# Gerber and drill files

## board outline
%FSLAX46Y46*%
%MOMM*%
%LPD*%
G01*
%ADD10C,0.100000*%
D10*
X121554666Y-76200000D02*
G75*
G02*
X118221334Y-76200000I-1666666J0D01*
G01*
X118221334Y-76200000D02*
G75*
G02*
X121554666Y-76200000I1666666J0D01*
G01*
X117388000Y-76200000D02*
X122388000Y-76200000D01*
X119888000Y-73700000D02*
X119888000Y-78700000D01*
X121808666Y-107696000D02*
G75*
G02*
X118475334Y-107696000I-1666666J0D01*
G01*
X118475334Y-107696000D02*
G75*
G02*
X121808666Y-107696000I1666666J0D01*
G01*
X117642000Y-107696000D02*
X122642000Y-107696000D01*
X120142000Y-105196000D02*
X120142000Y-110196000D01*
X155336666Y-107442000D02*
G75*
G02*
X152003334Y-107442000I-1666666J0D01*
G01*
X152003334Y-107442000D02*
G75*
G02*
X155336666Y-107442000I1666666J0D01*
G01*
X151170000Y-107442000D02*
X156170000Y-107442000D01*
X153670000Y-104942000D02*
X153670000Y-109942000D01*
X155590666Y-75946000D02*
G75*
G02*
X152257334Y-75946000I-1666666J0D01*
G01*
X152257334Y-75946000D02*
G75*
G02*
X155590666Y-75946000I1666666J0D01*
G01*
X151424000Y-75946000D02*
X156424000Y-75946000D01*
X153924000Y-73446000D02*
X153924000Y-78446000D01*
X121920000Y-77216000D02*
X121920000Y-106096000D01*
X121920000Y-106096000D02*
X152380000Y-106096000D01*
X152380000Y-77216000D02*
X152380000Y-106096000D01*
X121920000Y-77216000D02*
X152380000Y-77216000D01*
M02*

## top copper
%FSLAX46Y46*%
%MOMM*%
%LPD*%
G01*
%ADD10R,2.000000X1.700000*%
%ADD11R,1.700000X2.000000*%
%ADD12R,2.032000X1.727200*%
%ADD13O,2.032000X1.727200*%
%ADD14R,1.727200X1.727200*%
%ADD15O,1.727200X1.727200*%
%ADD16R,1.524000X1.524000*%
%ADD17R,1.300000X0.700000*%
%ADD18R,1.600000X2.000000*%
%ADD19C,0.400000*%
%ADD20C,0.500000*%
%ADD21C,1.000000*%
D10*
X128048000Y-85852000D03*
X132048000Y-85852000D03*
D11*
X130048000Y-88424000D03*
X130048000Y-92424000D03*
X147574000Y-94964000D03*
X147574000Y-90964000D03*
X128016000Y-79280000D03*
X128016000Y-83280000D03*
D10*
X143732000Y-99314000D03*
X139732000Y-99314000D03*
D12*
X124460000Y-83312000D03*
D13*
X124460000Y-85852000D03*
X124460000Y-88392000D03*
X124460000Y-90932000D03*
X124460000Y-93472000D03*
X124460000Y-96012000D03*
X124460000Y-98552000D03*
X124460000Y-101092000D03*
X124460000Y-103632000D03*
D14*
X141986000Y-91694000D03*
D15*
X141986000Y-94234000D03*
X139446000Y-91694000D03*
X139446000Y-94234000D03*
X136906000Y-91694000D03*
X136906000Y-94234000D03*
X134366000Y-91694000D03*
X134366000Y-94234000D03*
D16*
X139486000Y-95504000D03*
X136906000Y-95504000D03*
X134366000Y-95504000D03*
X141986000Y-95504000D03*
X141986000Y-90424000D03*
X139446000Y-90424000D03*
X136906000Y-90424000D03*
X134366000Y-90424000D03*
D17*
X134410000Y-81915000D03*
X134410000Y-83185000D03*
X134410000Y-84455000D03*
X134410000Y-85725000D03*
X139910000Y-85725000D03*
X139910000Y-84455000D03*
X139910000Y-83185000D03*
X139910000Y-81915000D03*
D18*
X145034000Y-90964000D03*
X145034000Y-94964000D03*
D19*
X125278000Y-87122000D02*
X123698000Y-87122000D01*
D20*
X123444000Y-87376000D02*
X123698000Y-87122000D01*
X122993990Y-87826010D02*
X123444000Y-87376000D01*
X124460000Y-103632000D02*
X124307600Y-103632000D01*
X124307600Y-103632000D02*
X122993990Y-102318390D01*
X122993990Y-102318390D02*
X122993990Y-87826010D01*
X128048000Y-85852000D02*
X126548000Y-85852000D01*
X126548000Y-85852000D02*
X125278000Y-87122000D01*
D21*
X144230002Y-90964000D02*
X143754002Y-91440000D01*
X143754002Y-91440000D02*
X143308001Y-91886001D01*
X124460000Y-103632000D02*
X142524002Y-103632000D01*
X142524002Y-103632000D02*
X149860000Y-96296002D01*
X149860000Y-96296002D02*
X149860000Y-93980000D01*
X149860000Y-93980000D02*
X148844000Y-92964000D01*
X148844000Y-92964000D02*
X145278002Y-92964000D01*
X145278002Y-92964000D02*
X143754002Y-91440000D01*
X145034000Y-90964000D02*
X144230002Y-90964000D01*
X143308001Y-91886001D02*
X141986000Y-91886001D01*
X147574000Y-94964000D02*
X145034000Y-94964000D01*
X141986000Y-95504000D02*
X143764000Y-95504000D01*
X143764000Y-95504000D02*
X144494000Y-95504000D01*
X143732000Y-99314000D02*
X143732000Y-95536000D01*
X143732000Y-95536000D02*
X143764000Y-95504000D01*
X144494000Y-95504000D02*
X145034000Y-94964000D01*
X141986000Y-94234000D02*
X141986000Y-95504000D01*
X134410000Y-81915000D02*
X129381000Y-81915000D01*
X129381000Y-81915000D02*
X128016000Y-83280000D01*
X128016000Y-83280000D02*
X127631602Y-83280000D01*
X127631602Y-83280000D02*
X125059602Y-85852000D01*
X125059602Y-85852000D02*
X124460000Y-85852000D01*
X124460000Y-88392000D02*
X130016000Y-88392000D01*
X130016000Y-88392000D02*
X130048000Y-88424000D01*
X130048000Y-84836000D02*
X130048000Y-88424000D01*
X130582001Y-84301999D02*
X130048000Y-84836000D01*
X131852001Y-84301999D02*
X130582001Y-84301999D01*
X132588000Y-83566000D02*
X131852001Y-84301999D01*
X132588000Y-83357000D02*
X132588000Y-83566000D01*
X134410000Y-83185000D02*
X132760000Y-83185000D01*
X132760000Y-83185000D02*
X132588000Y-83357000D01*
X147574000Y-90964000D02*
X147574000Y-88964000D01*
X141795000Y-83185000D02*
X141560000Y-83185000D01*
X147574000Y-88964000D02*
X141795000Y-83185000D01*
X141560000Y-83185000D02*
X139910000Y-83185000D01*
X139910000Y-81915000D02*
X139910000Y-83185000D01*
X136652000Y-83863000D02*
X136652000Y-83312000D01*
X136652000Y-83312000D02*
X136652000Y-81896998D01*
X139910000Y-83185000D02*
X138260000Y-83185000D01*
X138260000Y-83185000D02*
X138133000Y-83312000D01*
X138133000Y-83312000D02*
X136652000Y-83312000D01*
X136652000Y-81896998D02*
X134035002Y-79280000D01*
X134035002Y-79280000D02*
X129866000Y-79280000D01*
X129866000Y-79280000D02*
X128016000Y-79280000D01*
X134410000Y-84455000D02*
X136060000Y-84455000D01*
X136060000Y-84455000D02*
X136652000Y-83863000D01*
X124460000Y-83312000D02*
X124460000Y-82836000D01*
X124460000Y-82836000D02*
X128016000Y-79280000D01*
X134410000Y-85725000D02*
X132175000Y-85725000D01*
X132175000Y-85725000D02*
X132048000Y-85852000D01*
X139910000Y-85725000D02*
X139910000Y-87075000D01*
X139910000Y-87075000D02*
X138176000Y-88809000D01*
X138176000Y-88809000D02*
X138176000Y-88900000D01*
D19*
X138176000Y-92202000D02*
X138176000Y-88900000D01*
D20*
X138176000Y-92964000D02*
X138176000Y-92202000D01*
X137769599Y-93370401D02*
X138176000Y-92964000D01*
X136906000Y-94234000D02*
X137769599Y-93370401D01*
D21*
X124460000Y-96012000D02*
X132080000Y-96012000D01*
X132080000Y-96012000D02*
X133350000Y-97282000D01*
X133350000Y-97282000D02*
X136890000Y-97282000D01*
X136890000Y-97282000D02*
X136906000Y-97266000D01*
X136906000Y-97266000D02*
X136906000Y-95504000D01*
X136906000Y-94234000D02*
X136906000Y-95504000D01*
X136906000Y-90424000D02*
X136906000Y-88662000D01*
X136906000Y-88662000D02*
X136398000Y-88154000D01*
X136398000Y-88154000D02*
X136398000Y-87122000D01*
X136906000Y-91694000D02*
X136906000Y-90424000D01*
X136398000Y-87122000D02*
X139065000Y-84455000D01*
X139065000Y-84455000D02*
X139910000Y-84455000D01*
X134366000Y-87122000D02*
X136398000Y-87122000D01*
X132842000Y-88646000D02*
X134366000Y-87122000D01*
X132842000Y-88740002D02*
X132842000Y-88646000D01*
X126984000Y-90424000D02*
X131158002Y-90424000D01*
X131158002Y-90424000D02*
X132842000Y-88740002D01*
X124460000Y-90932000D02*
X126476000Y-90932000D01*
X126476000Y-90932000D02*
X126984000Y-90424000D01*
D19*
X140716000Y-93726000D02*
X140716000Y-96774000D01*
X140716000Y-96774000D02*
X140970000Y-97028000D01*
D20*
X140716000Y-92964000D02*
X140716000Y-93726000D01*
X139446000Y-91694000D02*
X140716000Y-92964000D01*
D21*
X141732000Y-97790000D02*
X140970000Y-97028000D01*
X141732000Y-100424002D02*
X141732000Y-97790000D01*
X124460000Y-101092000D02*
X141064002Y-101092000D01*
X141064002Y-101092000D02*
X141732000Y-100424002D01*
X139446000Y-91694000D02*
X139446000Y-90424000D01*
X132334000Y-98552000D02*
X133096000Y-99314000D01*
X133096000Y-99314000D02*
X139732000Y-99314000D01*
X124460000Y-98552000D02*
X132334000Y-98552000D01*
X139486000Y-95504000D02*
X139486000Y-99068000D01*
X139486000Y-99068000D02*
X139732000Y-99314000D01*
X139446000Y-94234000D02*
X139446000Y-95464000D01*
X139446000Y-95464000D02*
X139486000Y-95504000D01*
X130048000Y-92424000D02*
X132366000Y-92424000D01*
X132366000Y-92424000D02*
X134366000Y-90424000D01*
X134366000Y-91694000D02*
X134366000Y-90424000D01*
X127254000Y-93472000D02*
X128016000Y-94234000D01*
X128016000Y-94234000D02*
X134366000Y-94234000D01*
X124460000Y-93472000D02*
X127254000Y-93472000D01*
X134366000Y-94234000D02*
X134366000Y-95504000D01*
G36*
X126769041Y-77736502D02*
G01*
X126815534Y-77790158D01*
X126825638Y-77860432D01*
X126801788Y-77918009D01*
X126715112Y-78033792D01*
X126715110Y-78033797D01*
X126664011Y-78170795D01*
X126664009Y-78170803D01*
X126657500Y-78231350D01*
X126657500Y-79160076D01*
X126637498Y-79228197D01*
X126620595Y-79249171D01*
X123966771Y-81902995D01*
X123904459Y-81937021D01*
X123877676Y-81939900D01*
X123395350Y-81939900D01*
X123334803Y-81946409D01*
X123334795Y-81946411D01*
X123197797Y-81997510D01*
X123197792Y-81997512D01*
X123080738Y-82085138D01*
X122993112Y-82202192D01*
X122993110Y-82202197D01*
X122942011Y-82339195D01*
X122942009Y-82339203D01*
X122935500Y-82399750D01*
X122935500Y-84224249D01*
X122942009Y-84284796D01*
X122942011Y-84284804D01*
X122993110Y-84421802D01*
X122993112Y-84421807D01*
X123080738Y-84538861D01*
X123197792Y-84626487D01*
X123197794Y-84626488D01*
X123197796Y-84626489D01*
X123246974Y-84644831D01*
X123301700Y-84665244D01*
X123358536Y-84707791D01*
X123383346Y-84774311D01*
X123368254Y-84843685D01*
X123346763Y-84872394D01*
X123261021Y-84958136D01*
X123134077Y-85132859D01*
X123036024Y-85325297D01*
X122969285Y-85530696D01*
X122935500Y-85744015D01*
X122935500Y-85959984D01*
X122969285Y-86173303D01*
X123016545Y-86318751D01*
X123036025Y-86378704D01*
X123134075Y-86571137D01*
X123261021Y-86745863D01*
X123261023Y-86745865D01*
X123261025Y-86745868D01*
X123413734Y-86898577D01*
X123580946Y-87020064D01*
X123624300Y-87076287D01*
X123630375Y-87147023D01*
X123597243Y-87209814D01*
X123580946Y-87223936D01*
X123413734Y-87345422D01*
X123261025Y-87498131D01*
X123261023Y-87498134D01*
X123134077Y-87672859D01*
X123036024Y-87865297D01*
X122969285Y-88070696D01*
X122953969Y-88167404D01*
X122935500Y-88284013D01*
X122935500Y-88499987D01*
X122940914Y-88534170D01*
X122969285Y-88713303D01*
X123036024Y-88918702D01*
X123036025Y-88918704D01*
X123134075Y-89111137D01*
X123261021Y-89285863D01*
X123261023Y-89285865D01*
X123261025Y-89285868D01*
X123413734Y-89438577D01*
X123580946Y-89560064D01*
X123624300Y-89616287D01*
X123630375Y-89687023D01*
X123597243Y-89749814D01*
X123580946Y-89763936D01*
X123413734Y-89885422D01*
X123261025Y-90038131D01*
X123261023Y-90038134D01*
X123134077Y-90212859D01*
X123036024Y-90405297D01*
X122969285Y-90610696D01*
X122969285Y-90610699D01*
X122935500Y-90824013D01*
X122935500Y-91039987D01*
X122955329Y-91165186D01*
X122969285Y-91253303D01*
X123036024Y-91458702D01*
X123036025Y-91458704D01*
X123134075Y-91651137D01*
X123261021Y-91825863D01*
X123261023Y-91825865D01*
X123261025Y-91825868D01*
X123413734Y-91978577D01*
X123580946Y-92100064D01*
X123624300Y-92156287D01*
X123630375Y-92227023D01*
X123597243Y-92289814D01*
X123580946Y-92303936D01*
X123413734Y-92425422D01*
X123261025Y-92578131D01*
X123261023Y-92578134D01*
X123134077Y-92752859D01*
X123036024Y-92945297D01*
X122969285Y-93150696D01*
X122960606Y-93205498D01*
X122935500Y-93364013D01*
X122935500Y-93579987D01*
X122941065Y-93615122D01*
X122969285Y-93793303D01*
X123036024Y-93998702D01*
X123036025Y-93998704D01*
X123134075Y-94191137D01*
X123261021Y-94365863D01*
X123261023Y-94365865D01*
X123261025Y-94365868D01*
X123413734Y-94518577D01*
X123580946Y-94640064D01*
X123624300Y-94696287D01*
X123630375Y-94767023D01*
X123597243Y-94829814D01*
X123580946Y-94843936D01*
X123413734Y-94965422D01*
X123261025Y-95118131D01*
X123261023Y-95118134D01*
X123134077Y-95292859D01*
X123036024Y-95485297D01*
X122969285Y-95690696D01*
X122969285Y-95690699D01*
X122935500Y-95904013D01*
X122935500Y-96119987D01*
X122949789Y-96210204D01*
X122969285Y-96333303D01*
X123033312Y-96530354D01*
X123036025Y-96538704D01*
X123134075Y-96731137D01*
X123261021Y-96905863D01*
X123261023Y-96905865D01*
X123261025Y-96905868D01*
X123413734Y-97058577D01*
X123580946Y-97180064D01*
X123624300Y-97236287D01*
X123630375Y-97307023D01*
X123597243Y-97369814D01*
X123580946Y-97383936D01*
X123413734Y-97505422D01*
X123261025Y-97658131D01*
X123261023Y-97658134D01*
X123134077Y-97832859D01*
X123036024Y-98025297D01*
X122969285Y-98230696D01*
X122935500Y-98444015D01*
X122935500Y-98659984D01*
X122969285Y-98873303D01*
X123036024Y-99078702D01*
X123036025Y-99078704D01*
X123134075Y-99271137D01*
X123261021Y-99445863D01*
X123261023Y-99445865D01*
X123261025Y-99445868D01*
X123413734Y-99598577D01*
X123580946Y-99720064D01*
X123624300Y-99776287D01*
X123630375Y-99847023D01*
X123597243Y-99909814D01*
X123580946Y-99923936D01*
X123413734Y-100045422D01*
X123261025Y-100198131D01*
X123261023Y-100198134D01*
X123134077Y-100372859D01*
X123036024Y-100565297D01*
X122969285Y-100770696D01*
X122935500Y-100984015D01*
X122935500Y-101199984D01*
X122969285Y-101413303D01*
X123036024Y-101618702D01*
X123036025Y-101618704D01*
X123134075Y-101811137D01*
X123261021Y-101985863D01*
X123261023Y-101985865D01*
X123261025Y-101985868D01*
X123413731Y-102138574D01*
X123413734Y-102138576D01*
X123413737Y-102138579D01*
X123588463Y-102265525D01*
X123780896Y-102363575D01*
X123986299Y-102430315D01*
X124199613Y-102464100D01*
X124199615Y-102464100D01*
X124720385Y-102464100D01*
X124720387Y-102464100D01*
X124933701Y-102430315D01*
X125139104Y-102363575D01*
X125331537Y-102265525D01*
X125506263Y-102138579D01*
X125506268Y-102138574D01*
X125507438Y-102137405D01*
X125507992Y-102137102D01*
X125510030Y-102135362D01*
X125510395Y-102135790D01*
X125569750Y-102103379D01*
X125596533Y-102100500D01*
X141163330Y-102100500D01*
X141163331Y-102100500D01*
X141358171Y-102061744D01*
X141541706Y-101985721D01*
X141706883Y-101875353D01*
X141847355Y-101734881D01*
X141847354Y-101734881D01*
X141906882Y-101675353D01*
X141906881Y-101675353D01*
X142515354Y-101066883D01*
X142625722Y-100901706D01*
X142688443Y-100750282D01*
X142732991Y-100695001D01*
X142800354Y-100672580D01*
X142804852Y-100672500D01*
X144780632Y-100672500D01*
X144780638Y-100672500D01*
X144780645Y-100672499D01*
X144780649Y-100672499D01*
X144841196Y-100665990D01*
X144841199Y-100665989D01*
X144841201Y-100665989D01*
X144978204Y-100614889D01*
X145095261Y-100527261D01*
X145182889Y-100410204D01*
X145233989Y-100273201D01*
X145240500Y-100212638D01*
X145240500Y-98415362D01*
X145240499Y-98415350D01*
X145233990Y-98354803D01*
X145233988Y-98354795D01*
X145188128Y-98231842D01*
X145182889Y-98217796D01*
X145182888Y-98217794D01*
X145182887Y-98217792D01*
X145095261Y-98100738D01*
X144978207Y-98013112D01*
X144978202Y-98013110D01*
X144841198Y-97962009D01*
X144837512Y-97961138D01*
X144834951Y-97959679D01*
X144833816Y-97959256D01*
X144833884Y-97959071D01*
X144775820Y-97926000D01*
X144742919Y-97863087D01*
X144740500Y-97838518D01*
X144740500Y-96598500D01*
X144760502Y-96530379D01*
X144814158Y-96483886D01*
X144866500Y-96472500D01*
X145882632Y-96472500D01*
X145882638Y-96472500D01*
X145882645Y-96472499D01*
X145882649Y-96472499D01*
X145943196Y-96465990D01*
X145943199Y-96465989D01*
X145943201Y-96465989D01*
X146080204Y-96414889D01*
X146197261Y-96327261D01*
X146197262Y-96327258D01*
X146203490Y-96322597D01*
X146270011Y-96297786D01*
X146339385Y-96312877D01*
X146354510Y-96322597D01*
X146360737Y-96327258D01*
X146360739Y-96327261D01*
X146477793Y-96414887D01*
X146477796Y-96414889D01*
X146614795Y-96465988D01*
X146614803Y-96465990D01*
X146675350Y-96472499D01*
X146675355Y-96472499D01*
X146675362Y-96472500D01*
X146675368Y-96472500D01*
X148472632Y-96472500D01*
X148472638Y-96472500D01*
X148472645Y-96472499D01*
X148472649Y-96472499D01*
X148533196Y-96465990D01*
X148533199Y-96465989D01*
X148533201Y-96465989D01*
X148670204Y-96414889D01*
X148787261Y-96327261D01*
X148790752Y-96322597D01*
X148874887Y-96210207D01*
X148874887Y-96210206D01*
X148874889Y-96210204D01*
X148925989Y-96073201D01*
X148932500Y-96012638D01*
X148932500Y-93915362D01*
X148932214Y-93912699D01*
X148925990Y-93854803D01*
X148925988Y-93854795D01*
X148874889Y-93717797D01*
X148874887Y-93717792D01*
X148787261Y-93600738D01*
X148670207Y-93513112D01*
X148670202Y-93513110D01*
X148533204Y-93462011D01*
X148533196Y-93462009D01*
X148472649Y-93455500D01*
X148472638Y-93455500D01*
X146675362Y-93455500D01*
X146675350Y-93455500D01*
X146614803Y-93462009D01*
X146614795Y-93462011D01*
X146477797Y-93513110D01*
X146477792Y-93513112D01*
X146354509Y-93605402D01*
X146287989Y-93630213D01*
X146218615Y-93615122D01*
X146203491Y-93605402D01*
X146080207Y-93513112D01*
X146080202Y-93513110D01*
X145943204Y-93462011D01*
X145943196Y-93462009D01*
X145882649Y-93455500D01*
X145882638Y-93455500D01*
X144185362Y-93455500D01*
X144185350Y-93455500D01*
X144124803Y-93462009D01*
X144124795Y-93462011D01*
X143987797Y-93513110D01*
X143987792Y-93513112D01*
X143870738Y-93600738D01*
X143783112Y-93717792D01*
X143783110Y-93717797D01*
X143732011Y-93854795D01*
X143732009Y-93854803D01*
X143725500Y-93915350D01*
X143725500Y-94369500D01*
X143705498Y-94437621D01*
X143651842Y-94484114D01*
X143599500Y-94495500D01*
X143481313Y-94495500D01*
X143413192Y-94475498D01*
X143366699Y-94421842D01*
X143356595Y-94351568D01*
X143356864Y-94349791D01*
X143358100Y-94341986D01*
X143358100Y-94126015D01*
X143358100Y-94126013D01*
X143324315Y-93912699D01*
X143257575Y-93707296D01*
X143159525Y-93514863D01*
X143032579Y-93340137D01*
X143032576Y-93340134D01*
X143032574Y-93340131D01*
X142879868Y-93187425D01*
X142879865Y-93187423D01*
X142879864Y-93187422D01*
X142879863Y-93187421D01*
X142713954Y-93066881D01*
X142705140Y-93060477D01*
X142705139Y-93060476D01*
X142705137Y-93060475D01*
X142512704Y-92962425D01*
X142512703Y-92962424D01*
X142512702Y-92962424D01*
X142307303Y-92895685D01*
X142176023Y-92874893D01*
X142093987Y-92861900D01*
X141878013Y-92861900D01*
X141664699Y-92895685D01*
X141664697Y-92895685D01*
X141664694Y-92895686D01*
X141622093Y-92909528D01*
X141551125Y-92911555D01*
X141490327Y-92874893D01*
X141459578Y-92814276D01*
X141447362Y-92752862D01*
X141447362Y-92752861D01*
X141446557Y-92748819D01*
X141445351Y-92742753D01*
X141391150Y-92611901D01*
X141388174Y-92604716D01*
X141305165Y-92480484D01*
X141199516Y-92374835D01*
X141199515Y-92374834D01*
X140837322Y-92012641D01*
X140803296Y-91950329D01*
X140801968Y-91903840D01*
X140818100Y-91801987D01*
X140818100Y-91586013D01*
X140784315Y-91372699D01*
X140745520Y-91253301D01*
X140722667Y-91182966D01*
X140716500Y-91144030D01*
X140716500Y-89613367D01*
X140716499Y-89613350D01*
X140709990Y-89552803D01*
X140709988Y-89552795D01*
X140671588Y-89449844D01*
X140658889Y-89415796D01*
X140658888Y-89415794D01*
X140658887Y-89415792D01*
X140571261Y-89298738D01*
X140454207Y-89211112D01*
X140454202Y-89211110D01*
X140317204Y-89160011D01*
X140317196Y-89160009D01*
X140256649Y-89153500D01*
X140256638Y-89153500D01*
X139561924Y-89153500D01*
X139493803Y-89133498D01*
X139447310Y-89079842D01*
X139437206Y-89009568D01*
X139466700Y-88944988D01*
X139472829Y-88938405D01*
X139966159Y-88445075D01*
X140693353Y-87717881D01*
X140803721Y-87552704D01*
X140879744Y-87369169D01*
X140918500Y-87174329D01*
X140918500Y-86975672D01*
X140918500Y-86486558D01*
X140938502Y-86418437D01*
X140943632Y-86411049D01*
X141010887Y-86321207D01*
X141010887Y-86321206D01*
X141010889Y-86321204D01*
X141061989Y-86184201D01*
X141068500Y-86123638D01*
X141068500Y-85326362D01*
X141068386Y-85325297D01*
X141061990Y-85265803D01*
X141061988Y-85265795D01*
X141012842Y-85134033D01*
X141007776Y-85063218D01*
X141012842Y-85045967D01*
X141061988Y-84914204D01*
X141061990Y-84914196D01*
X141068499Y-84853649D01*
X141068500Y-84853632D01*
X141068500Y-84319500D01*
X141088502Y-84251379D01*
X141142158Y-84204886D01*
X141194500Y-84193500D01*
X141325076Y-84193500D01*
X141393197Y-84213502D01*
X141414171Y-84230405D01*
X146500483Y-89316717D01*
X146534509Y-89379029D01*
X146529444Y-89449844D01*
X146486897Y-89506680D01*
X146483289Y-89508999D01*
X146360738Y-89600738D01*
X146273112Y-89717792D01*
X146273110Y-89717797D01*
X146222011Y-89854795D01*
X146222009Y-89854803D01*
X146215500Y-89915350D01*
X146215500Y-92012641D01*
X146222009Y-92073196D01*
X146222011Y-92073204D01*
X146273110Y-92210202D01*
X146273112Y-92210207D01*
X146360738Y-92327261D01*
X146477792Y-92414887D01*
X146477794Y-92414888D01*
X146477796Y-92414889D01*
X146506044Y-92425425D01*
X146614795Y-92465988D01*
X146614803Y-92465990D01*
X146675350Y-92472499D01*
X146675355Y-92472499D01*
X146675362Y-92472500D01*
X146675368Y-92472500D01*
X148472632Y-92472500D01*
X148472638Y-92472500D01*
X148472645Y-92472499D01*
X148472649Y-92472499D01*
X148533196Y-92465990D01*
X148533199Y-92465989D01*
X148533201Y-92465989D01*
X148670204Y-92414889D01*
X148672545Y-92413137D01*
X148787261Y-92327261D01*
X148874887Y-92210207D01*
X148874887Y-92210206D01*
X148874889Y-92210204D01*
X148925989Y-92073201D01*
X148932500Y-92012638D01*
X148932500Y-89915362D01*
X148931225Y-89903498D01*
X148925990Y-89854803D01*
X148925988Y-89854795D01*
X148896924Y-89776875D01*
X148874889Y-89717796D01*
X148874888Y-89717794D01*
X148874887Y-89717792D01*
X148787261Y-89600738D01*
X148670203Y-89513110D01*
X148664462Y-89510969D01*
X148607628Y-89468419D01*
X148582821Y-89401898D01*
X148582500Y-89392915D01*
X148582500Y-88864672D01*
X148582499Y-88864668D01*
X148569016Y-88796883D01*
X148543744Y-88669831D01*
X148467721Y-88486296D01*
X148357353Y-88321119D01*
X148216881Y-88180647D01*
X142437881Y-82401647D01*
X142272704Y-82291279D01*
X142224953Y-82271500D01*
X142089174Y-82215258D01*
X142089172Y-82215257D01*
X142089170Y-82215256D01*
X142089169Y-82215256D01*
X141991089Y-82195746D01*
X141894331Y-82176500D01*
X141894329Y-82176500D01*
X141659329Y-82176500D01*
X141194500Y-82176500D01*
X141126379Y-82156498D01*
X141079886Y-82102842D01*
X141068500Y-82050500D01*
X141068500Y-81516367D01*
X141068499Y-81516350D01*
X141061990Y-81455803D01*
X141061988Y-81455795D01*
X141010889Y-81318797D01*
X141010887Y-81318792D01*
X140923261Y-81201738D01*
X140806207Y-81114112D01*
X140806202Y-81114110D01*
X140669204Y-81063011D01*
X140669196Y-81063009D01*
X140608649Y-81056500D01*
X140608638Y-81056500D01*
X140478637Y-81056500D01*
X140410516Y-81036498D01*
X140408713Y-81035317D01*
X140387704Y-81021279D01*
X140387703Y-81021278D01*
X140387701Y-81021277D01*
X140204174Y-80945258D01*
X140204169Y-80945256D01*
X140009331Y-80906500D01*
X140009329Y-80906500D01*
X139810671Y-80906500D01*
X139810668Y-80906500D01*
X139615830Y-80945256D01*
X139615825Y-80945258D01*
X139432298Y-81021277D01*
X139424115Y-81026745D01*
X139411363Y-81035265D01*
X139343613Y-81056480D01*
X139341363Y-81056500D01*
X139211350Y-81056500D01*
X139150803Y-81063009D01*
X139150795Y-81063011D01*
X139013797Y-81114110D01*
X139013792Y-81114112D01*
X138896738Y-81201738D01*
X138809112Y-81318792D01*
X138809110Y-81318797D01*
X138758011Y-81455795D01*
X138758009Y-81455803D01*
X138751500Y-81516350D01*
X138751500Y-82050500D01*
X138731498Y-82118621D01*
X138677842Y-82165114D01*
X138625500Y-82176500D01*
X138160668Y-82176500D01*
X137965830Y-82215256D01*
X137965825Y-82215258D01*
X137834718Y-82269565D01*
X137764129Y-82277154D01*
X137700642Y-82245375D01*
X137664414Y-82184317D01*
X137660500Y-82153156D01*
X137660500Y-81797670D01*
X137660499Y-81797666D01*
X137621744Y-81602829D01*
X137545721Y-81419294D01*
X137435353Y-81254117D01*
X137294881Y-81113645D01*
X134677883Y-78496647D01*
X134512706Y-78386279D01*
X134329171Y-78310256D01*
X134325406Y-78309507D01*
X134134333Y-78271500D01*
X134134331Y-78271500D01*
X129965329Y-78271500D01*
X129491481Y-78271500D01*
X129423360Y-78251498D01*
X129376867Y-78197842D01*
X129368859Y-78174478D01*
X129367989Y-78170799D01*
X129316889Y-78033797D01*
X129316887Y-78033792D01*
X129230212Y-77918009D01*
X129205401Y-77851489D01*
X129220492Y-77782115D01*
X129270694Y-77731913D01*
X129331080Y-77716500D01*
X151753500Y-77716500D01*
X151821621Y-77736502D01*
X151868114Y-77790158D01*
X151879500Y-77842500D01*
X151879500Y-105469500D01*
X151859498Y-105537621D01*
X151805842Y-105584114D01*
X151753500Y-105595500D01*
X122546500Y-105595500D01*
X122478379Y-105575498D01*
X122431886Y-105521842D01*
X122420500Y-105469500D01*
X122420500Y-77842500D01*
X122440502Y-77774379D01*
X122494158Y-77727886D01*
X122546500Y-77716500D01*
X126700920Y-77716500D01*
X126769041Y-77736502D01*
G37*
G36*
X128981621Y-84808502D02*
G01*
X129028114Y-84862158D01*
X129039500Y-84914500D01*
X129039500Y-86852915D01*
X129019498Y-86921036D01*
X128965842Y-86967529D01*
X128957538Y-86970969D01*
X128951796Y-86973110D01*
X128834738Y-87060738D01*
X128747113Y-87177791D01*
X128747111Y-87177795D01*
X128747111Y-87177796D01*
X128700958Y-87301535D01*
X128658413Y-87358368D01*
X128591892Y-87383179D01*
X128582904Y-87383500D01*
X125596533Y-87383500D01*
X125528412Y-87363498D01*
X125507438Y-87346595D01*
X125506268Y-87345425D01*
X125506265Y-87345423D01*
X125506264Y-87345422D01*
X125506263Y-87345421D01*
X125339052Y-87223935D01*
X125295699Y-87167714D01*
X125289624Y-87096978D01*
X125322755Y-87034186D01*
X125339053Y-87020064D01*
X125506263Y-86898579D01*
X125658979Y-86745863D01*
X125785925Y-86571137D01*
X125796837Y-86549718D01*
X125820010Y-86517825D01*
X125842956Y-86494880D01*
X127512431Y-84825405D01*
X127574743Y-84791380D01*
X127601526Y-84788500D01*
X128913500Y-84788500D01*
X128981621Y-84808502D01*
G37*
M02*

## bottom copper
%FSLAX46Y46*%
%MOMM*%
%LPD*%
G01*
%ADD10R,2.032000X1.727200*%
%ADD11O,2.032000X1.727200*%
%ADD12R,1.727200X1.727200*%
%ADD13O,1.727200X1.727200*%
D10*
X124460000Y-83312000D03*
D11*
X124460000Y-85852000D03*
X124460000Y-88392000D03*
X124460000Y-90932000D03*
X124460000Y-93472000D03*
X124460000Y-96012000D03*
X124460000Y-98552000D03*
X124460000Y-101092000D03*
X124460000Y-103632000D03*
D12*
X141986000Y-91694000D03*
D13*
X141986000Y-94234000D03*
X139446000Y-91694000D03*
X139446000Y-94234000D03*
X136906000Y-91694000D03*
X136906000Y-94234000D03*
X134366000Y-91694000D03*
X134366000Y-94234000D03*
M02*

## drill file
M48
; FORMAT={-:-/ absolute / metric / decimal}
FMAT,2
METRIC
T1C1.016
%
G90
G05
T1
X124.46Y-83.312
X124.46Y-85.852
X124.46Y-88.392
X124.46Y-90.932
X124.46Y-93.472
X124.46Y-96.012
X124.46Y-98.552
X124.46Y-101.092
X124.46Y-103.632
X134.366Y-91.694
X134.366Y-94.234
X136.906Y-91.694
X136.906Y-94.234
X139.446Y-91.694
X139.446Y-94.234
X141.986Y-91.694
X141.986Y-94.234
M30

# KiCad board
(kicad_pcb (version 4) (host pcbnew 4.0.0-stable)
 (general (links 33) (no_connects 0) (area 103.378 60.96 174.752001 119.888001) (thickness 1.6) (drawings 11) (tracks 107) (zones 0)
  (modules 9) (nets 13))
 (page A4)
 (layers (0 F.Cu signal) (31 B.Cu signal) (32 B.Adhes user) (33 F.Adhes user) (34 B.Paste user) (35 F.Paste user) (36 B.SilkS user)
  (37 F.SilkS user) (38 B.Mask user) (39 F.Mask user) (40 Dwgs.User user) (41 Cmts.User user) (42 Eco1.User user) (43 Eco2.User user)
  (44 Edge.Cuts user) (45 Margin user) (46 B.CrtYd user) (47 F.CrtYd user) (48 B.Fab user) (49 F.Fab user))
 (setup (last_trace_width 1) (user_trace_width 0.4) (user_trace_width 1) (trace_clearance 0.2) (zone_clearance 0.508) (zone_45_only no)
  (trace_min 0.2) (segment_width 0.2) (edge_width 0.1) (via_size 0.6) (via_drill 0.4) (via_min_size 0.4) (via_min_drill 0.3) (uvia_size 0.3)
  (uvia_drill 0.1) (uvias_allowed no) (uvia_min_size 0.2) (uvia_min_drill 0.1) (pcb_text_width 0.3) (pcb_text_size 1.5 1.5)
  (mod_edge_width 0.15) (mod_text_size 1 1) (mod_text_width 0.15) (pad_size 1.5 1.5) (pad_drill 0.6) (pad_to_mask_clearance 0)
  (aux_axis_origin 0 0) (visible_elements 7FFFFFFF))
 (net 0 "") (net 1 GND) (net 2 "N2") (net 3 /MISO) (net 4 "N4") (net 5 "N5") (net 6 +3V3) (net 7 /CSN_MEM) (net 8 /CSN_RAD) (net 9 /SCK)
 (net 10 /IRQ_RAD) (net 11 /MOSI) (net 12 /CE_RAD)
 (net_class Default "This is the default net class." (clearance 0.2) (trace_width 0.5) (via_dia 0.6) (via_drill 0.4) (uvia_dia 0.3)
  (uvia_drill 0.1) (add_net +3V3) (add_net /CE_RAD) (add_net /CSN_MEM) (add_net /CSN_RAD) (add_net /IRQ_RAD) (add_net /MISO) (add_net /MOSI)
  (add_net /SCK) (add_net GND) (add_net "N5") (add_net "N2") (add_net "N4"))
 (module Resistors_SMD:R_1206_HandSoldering (layer F.Cu) (at 130.048 85.852)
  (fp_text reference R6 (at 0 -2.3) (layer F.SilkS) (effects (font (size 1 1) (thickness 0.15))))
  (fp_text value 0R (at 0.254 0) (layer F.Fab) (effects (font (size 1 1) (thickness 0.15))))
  (pad 1 smd rect (at -2 0) (size 2 1.7) (layers F.Cu F.Paste F.Mask) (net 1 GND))
  (pad 2 smd rect (at 2 0) (size 2 1.7) (layers F.Cu F.Paste F.Mask) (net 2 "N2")))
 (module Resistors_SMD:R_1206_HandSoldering (layer F.Cu) (at 130.048 90.424 270)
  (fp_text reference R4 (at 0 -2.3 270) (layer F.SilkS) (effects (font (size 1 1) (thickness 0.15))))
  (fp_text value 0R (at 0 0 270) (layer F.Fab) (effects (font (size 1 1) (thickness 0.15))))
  (pad 1 smd rect (at -2 0 270) (size 2 1.7) (layers F.Cu F.Paste F.Mask) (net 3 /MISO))
  (pad 2 smd rect (at 2 0 270) (size 2 1.7) (layers F.Cu F.Paste F.Mask) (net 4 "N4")))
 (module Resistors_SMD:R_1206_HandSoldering (layer F.Cu) (at 147.574 92.964 90)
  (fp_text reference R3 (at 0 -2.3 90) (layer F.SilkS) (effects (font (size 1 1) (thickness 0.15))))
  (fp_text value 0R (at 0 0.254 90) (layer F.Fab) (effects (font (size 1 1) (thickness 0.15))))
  (pad 1 smd rect (at -2 0 90) (size 2 1.7) (layers F.Cu F.Paste F.Mask) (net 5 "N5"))
  (pad 2 smd rect (at 2 0 90) (size 2 1.7) (layers F.Cu F.Paste F.Mask) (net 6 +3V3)))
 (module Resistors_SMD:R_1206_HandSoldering (layer F.Cu) (at 128.016 81.28 270)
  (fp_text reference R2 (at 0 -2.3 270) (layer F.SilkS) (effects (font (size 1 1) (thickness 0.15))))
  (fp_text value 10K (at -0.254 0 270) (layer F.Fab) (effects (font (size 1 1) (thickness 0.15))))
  (pad 1 smd rect (at -2 0 270) (size 2 1.7) (layers F.Cu F.Paste F.Mask) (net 6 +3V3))
  (pad 2 smd rect (at 2 0 270) (size 2 1.7) (layers F.Cu F.Paste F.Mask) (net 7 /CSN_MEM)))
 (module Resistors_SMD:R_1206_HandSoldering (layer F.Cu) (at 141.732 99.314 180)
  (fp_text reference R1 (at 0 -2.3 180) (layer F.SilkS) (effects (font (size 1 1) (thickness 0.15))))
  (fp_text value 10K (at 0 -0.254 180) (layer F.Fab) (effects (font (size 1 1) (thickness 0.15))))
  (pad 1 smd rect (at -2 0 180) (size 2 1.7) (layers F.Cu F.Paste F.Mask) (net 5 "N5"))
  (pad 2 smd rect (at 2 0 180) (size 2 1.7) (layers F.Cu F.Paste F.Mask) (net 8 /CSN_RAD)))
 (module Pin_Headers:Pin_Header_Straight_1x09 (layer F.Cu) (at 124.46 83.312)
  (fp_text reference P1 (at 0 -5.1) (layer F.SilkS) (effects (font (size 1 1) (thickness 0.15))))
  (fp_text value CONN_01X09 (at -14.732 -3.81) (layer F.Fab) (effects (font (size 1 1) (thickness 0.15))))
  (pad 1 thru_hole rect (at 0 0) (size 2.032 1.7272) (drill 1.016) (layers *.Cu *.Mask F.SilkS) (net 6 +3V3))
  (pad 2 thru_hole oval (at 0 2.54) (size 2.032 1.7272) (drill 1.016) (layers *.Cu *.Mask F.SilkS) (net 7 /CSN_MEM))
  (pad 3 thru_hole oval (at 0 5.08) (size 2.032 1.7272) (drill 1.016) (layers *.Cu *.Mask F.SilkS) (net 3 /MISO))
  (pad 4 thru_hole oval (at 0 7.62) (size 2.032 1.7272) (drill 1.016) (layers *.Cu *.Mask F.SilkS) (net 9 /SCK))
  (pad 5 thru_hole oval (at 0 10.16) (size 2.032 1.7272) (drill 1.016) (layers *.Cu *.Mask F.SilkS) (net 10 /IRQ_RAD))
  (pad 6 thru_hole oval (at 0 12.7) (size 2.032 1.7272) (drill 1.016) (layers *.Cu *.Mask F.SilkS) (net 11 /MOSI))
  (pad 7 thru_hole oval (at 0 15.24) (size 2.032 1.7272) (drill 1.016) (layers *.Cu *.Mask F.SilkS) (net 8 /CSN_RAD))
  (pad 8 thru_hole oval (at 0 17.78) (size 2.032 1.7272) (drill 1.016) (layers *.Cu *.Mask F.SilkS) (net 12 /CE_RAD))
  (pad 9 thru_hole oval (at 0 20.32) (size 2.032 1.7272) (drill 1.016) (layers *.Cu *.Mask F.SilkS) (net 1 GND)))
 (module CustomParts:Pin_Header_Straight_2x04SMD (layer F.Cu) (at 141.986 91.694 270)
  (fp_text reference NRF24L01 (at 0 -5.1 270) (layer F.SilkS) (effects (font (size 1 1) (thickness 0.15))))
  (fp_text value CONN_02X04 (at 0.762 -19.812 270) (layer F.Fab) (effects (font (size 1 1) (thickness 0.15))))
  (pad 1 thru_hole rect (at 0 0 270) (size 1.7272 1.7272) (drill 1.016) (layers *.Cu *.Mask F.SilkS) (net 1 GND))
  (pad 2 thru_hole oval (at 2.54 0 270) (size 1.7272 1.7272) (drill 1.016) (layers *.Cu *.Mask F.SilkS) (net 5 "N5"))
  (pad 3 thru_hole oval (at 0 2.54 270) (size 1.7272 1.7272) (drill 1.016) (layers *.Cu *.Mask F.SilkS) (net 12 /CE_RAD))
  (pad 4 thru_hole oval (at 2.54 2.54 270) (size 1.7272 1.7272) (drill 1.016) (layers *.Cu *.Mask F.SilkS) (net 8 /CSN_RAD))
  (pad 5 thru_hole oval (at 0 5.08 270) (size 1.7272 1.7272) (drill 1.016) (layers *.Cu *.Mask F.SilkS) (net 9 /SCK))
  (pad 6 thru_hole oval (at 2.54 5.08 270) (size 1.7272 1.7272) (drill 1.016) (layers *.Cu *.Mask F.SilkS) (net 11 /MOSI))
  (pad 7 thru_hole oval (at 0 7.62 270) (size 1.7272 1.7272) (drill 1.016) (layers *.Cu *.Mask F.SilkS) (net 4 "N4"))
  (pad 8 thru_hole oval (at 2.54 7.62 270) (size 1.7272 1.7272) (drill 1.016) (layers *.Cu *.Mask F.SilkS) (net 10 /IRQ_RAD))
  (pad 4 smd rect (at 3.81 2.5 270) (size 1.524 1.524) (layers F.Cu F.Paste F.Mask) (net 8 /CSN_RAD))
  (pad 6 smd rect (at 3.81 5.08 270) (size 1.524 1.524) (layers F.Cu F.Paste F.Mask) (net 11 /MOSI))
  (pad 8 smd rect (at 3.81 7.62 270) (size 1.524 1.524) (layers F.Cu F.Paste F.Mask) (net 10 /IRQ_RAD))
  (pad 2 smd rect (at 3.81 0 270) (size 1.524 1.524) (layers F.Cu F.Paste F.Mask) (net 5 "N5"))
  (pad 1 smd rect (at -1.27 0 270) (size 1.524 1.524) (layers F.Cu F.Paste F.Mask) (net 1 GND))
  (pad 3 smd rect (at -1.27 2.54 270) (size 1.524 1.524) (layers F.Cu F.Paste F.Mask) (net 12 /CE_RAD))
  (pad 5 smd rect (at -1.27 5.08 270) (size 1.524 1.524) (layers F.Cu F.Paste F.Mask) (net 9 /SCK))
  (pad 7 smd rect (at -1.27 7.62 270) (size 1.524 1.524) (layers F.Cu F.Paste F.Mask) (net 4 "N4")))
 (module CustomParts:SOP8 (layer F.Cu) (at 137.16 83.82)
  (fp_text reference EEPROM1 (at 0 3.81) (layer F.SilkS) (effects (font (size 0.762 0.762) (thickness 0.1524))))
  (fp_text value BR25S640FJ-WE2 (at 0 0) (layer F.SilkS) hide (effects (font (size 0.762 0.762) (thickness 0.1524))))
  (pad 1 smd rect (at -2.75 -1.905) (size 1.3 0.7) (layers F.Cu F.Paste F.Mask) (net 7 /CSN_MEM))
  (pad 2 smd rect (at -2.75 -0.635) (size 1.3 0.7) (layers F.Cu F.Paste F.Mask) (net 3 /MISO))
  (pad 3 smd rect (at -2.75 0.635) (size 1.3 0.7) (layers F.Cu F.Paste F.Mask) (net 6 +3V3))
  (pad 4 smd rect (at -2.75 1.905) (size 1.3 0.7) (layers F.Cu F.Paste F.Mask) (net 2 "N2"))
  (pad 5 smd rect (at 2.75 1.905) (size 1.3 0.7) (layers F.Cu F.Paste F.Mask) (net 11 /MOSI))
  (pad 6 smd rect (at 2.75 0.635) (size 1.3 0.7) (layers F.Cu F.Paste F.Mask) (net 9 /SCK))
  (pad 7 smd rect (at 2.75 -0.635) (size 1.3 0.7) (layers F.Cu F.Paste F.Mask) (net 6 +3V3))
  (pad 8 smd rect (at 2.75 -1.905) (size 1.3 0.7) (layers F.Cu F.Paste F.Mask) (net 6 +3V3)))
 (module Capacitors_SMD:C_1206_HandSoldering (layer F.Cu) (at 145.034 92.964 270)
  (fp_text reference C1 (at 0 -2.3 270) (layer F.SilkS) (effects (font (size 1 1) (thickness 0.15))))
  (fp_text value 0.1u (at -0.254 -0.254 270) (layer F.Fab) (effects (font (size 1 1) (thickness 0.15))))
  (pad 1 smd rect (at -2 0 270) (size 2 1.6) (layers F.Cu F.Paste F.Mask) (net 1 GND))
  (pad 2 smd rect (at 2 0 270) (size 2 1.6) (layers F.Cu F.Paste F.Mask) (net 5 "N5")))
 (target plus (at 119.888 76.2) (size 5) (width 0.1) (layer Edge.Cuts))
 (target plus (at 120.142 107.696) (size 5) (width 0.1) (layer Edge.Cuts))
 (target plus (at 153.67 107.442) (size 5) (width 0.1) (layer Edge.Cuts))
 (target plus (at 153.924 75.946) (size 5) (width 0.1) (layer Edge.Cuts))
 (gr_line (start 121.92 77.216) (end 121.92 106.096) (layer Edge.Cuts) (width 0.1))
 (gr_line (start 121.92 106.096) (end 152.38 106.096) (layer Edge.Cuts) (width 0.1))
 (gr_line (start 152.38 77.216) (end 152.38 106.096) (layer Edge.Cuts) (width 0.1))
 (gr_line (start 121.92 77.216) (end 152.38 77.216) (layer Edge.Cuts) (width 0.1))
 (segment (start 125.278 87.122) (end 123.698 87.122) (width 0.4) (layer F.Cu) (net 1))
 (segment (start 123.444 87.376) (end 123.698 87.122) (width 0.5) (layer F.Cu) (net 1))
 (segment (start 122.99399 87.82601) (end 123.444 87.376) (width 0.5) (layer F.Cu) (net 1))
 (segment (start 124.46 103.632) (end 124.3076 103.632) (width 0.5) (layer F.Cu) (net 1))
 (segment (start 124.3076 103.632) (end 122.99399 102.31839) (width 0.5) (layer F.Cu) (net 1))
 (segment (start 122.99399 102.31839) (end 122.99399 87.82601) (width 0.5) (layer F.Cu) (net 1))
 (segment (start 128.048 85.852) (end 126.548 85.852) (width 0.5) (layer F.Cu) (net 1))
 (segment (start 126.548 85.852) (end 125.278 87.122) (width 0.5) (layer F.Cu) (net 1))
 (segment (start 144.230002 90.964) (end 143.754002 91.44) (width 1) (layer F.Cu) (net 1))
 (segment (start 143.754002 91.44) (end 143.308001 91.886001) (width 1) (layer F.Cu) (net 1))
 (segment (start 124.46 103.632) (end 142.524002 103.632) (width 1) (layer F.Cu) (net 1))
 (segment (start 142.524002 103.632) (end 149.86 96.296002) (width 1) (layer F.Cu) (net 1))
 (segment (start 149.86 96.296002) (end 149.86 93.98) (width 1) (layer F.Cu) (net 1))
 (segment (start 149.86 93.98) (end 148.844 92.964) (width 1) (layer F.Cu) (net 1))
 (segment (start 148.844 92.964) (end 145.278002 92.964) (width 1) (layer F.Cu) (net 1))
 (segment (start 145.278002 92.964) (end 143.754002 91.44) (width 1) (layer F.Cu) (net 1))
 (segment (start 145.034 90.964) (end 144.230002 90.964) (width 1) (layer F.Cu) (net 1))
 (segment (start 143.308001 91.886001) (end 141.986 91.886001) (width 1) (layer F.Cu) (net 1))
 (segment (start 147.574 94.964) (end 145.034 94.964) (width 1) (layer F.Cu) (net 5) (status C00000))
 (segment (start 141.986 95.504) (end 143.764 95.504) (width 1) (layer F.Cu) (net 5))
 (segment (start 143.764 95.504) (end 144.494 95.504) (width 1) (layer F.Cu) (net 5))
 (segment (start 143.732 99.314) (end 143.732 95.536) (width 1) (layer F.Cu) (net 5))
 (segment (start 143.732 95.536) (end 143.764 95.504) (width 1) (layer F.Cu) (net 5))
 (segment (start 144.494 95.504) (end 145.034 94.964) (width 1) (layer F.Cu) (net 5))
 (segment (start 141.986 94.234) (end 141.986 95.504) (width 1) (layer F.Cu) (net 5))
 (segment (start 134.41 81.915) (end 129.381 81.915) (width 1) (layer F.Cu) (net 7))
 (segment (start 129.381 81.915) (end 128.016 83.28) (width 1) (layer F.Cu) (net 7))
 (segment (start 128.016 83.28) (end 127.631602 83.28) (width 1) (layer F.Cu) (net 7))
 (segment (start 127.631602 83.28) (end 125.059602 85.852) (width 1) (layer F.Cu) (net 7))
 (segment (start 125.059602 85.852) (end 124.46 85.852) (width 1) (layer F.Cu) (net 7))
 (segment (start 124.46 88.392) (end 130.016 88.392) (width 1) (layer F.Cu) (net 3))
 (segment (start 130.016 88.392) (end 130.048 88.424) (width 1) (layer F.Cu) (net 3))
 (segment (start 130.048 84.836) (end 130.048 88.424) (width 1) (layer F.Cu) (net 3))
 (segment (start 130.582001 84.301999) (end 130.048 84.836) (width 1) (layer F.Cu) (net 3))
 (segment (start 131.852001 84.301999) (end 130.582001 84.301999) (width 1) (layer F.Cu) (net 3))
 (segment (start 132.588 83.566) (end 131.852001 84.301999) (width 1) (layer F.Cu) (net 3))
 (segment (start 132.588 83.357) (end 132.588 83.566) (width 1) (layer F.Cu) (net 3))
 (segment (start 134.41 83.185) (end 132.76 83.185) (width 1) (layer F.Cu) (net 3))
 (segment (start 132.76 83.185) (end 132.588 83.357) (width 1) (layer F.Cu) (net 3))
 (segment (start 147.574 90.964) (end 147.574 88.964) (width 1) (layer F.Cu) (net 6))
 (segment (start 141.795 83.185) (end 141.56 83.185) (width 1) (layer F.Cu) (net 6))
 (segment (start 147.574 88.964) (end 141.795 83.185) (width 1) (layer F.Cu) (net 6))
 (segment (start 141.56 83.185) (end 139.91 83.185) (width 1) (layer F.Cu) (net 6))
 (segment (start 139.91 81.915) (end 139.91 83.185) (width 1) (layer F.Cu) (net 6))
 (segment (start 136.652 83.863) (end 136.652 83.312) (width 1) (layer F.Cu) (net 6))
 (segment (start 136.652 83.312) (end 136.652 81.896998) (width 1) (layer F.Cu) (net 6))
 (segment (start 139.91 83.185) (end 138.26 83.185) (width 1) (layer F.Cu) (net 6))
 (segment (start 138.26 83.185) (end 138.133 83.312) (width 1) (layer F.Cu) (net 6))
 (segment (start 138.133 83.312) (end 136.652 83.312) (width 1) (layer F.Cu) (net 6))
 (segment (start 136.652 81.896998) (end 134.035002 79.28) (width 1) (layer F.Cu) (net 6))
 (segment (start 134.035002 79.28) (end 129.866 79.28) (width 1) (layer F.Cu) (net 6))
 (segment (start 129.866 79.28) (end 128.016 79.28) (width 1) (layer F.Cu) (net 6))
 (segment (start 134.41 84.455) (end 136.06 84.455) (width 1) (layer F.Cu) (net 6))
 (segment (start 136.06 84.455) (end 136.652 83.863) (width 1) (layer F.Cu) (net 6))
 (segment (start 124.46 83.312) (end 124.46 82.836) (width 1) (layer F.Cu) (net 6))
 (segment (start 124.46 82.836) (end 128.016 79.28) (width 1) (layer F.Cu) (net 6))
 (segment (start 134.41 85.725) (end 132.175 85.725) (width 1) (layer F.Cu) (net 2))
 (segment (start 132.175 85.725) (end 132.048 85.852) (width 1) (layer F.Cu) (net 2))
 (segment (start 139.91 85.725) (end 139.91 87.075) (width 1) (layer F.Cu) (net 11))
 (segment (start 139.91 87.075) (end 138.176 88.809) (width 1) (layer F.Cu) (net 11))
 (segment (start 138.176 88.809) (end 138.176 88.9) (width 1) (layer F.Cu) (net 11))
 (segment (start 138.176 92.202) (end 138.176 88.9) (width 0.4) (layer F.Cu) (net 11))
 (segment (start 138.176 92.964) (end 138.176 92.202) (width 0.5) (layer F.Cu) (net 11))
 (segment (start 137.769599 93.370401) (end 138.176 92.964) (width 0.5) (layer F.Cu) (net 11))
 (segment (start 136.906 94.234) (end 137.769599 93.370401) (width 0.5) (layer F.Cu) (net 11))
 (segment (start 124.46 96.012) (end 132.08 96.012) (width 1) (layer F.Cu) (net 11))
 (segment (start 132.08 96.012) (end 133.35 97.282) (width 1) (layer F.Cu) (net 11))
 (segment (start 133.35 97.282) (end 136.89 97.282) (width 1) (layer F.Cu) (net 11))
 (segment (start 136.89 97.282) (end 136.906 97.266) (width 1) (layer F.Cu) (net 11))
 (segment (start 136.906 97.266) (end 136.906 95.504) (width 1) (layer F.Cu) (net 11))
 (segment (start 136.906 94.234) (end 136.906 95.504) (width 1) (layer F.Cu) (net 11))
 (segment (start 136.906 90.424) (end 136.906 88.662) (width 1) (layer F.Cu) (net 9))
 (segment (start 136.906 88.662) (end 136.398 88.154) (width 1) (layer F.Cu) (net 9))
 (segment (start 136.398 88.154) (end 136.398 87.122) (width 1) (layer F.Cu) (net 9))
 (segment (start 136.906 91.694) (end 136.906 90.424) (width 1) (layer F.Cu) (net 9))
 (segment (start 136.398 87.122) (end 139.065 84.455) (width 1) (layer F.Cu) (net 9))
 (segment (start 139.065 84.455) (end 139.91 84.455) (width 1) (layer F.Cu) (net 9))
 (segment (start 134.366 87.122) (end 136.398 87.122) (width 1) (layer F.Cu) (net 9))
 (segment (start 132.842 88.646) (end 134.366 87.122) (width 1) (layer F.Cu) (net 9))
 (segment (start 132.842 88.740002) (end 132.842 88.646) (width 1) (layer F.Cu) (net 9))
 (segment (start 126.984 90.424) (end 131.158002 90.424) (width 1) (layer F.Cu) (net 9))
 (segment (start 131.158002 90.424) (end 132.842 88.740002) (width 1) (layer F.Cu) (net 9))
 (segment (start 124.46 90.932) (end 126.476 90.932) (width 1) (layer F.Cu) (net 9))
 (segment (start 126.476 90.932) (end 126.984 90.424) (width 1) (layer F.Cu) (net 9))
 (segment (start 140.716 93.726) (end 140.716 96.774) (width 0.4) (layer F.Cu) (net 12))
 (segment (start 140.716 96.774) (end 140.97 97.028) (width 0.4) (layer F.Cu) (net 12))
 (segment (start 140.716 92.964) (end 140.716 93.726) (width 0.5) (layer F.Cu) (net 12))
 (segment (start 139.446 91.694) (end 140.716 92.964) (width 0.5) (layer F.Cu) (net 12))
 (segment (start 141.732 97.79) (end 140.97 97.028) (width 1) (layer F.Cu) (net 12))
 (segment (start 141.732 100.424002) (end 141.732 97.79) (width 1) (layer F.Cu) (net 12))
 (segment (start 124.46 101.092) (end 141.064002 101.092) (width 1) (layer F.Cu) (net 12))
 (segment (start 141.064002 101.092) (end 141.732 100.424002) (width 1) (layer F.Cu) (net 12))
 (segment (start 139.446 91.694) (end 139.446 90.424) (width 1) (layer F.Cu) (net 12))
 (segment (start 132.334 98.552) (end 133.096 99.314) (width 1) (layer F.Cu) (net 8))
 (segment (start 133.096 99.314) (end 139.732 99.314) (width 1) (layer F.Cu) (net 8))
 (segment (start 124.46 98.552) (end 132.334 98.552) (width 1) (layer F.Cu) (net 8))
 (segment (start 139.486 95.504) (end 139.486 99.068) (width 1) (layer F.Cu) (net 8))
 (segment (start 139.486 99.068) (end 139.732 99.314) (width 1) (layer F.Cu) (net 8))
 (segment (start 139.446 94.234) (end 139.446 95.464) (width 1) (layer F.Cu) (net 8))
 (segment (start 139.446 95.464) (end 139.486 95.504) (width 1) (layer F.Cu) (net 8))
 (segment (start 130.048 92.424) (end 132.366 92.424) (width 1) (layer F.Cu) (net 4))
 (segment (start 132.366 92.424) (end 134.366 90.424) (width 1) (layer F.Cu) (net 4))
 (segment (start 134.366 91.694) (end 134.366 90.424) (width 1) (layer F.Cu) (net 4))
 (segment (start 127.254 93.472) (end 128.016 94.234) (width 1) (layer F.Cu) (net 10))
 (segment (start 128.016 94.234) (end 134.366 94.234) (width 1) (layer F.Cu) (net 10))
 (segment (start 124.46 93.472) (end 127.254 93.472) (width 1) (layer F.Cu) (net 10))
 (segment (start 134.366 94.234) (end 134.366 95.504) (width 1) (layer F.Cu) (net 10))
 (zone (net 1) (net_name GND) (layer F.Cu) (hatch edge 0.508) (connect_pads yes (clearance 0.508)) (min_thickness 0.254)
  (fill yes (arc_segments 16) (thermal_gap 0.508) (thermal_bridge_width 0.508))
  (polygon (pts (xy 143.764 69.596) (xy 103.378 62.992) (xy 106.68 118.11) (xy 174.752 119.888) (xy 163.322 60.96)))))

